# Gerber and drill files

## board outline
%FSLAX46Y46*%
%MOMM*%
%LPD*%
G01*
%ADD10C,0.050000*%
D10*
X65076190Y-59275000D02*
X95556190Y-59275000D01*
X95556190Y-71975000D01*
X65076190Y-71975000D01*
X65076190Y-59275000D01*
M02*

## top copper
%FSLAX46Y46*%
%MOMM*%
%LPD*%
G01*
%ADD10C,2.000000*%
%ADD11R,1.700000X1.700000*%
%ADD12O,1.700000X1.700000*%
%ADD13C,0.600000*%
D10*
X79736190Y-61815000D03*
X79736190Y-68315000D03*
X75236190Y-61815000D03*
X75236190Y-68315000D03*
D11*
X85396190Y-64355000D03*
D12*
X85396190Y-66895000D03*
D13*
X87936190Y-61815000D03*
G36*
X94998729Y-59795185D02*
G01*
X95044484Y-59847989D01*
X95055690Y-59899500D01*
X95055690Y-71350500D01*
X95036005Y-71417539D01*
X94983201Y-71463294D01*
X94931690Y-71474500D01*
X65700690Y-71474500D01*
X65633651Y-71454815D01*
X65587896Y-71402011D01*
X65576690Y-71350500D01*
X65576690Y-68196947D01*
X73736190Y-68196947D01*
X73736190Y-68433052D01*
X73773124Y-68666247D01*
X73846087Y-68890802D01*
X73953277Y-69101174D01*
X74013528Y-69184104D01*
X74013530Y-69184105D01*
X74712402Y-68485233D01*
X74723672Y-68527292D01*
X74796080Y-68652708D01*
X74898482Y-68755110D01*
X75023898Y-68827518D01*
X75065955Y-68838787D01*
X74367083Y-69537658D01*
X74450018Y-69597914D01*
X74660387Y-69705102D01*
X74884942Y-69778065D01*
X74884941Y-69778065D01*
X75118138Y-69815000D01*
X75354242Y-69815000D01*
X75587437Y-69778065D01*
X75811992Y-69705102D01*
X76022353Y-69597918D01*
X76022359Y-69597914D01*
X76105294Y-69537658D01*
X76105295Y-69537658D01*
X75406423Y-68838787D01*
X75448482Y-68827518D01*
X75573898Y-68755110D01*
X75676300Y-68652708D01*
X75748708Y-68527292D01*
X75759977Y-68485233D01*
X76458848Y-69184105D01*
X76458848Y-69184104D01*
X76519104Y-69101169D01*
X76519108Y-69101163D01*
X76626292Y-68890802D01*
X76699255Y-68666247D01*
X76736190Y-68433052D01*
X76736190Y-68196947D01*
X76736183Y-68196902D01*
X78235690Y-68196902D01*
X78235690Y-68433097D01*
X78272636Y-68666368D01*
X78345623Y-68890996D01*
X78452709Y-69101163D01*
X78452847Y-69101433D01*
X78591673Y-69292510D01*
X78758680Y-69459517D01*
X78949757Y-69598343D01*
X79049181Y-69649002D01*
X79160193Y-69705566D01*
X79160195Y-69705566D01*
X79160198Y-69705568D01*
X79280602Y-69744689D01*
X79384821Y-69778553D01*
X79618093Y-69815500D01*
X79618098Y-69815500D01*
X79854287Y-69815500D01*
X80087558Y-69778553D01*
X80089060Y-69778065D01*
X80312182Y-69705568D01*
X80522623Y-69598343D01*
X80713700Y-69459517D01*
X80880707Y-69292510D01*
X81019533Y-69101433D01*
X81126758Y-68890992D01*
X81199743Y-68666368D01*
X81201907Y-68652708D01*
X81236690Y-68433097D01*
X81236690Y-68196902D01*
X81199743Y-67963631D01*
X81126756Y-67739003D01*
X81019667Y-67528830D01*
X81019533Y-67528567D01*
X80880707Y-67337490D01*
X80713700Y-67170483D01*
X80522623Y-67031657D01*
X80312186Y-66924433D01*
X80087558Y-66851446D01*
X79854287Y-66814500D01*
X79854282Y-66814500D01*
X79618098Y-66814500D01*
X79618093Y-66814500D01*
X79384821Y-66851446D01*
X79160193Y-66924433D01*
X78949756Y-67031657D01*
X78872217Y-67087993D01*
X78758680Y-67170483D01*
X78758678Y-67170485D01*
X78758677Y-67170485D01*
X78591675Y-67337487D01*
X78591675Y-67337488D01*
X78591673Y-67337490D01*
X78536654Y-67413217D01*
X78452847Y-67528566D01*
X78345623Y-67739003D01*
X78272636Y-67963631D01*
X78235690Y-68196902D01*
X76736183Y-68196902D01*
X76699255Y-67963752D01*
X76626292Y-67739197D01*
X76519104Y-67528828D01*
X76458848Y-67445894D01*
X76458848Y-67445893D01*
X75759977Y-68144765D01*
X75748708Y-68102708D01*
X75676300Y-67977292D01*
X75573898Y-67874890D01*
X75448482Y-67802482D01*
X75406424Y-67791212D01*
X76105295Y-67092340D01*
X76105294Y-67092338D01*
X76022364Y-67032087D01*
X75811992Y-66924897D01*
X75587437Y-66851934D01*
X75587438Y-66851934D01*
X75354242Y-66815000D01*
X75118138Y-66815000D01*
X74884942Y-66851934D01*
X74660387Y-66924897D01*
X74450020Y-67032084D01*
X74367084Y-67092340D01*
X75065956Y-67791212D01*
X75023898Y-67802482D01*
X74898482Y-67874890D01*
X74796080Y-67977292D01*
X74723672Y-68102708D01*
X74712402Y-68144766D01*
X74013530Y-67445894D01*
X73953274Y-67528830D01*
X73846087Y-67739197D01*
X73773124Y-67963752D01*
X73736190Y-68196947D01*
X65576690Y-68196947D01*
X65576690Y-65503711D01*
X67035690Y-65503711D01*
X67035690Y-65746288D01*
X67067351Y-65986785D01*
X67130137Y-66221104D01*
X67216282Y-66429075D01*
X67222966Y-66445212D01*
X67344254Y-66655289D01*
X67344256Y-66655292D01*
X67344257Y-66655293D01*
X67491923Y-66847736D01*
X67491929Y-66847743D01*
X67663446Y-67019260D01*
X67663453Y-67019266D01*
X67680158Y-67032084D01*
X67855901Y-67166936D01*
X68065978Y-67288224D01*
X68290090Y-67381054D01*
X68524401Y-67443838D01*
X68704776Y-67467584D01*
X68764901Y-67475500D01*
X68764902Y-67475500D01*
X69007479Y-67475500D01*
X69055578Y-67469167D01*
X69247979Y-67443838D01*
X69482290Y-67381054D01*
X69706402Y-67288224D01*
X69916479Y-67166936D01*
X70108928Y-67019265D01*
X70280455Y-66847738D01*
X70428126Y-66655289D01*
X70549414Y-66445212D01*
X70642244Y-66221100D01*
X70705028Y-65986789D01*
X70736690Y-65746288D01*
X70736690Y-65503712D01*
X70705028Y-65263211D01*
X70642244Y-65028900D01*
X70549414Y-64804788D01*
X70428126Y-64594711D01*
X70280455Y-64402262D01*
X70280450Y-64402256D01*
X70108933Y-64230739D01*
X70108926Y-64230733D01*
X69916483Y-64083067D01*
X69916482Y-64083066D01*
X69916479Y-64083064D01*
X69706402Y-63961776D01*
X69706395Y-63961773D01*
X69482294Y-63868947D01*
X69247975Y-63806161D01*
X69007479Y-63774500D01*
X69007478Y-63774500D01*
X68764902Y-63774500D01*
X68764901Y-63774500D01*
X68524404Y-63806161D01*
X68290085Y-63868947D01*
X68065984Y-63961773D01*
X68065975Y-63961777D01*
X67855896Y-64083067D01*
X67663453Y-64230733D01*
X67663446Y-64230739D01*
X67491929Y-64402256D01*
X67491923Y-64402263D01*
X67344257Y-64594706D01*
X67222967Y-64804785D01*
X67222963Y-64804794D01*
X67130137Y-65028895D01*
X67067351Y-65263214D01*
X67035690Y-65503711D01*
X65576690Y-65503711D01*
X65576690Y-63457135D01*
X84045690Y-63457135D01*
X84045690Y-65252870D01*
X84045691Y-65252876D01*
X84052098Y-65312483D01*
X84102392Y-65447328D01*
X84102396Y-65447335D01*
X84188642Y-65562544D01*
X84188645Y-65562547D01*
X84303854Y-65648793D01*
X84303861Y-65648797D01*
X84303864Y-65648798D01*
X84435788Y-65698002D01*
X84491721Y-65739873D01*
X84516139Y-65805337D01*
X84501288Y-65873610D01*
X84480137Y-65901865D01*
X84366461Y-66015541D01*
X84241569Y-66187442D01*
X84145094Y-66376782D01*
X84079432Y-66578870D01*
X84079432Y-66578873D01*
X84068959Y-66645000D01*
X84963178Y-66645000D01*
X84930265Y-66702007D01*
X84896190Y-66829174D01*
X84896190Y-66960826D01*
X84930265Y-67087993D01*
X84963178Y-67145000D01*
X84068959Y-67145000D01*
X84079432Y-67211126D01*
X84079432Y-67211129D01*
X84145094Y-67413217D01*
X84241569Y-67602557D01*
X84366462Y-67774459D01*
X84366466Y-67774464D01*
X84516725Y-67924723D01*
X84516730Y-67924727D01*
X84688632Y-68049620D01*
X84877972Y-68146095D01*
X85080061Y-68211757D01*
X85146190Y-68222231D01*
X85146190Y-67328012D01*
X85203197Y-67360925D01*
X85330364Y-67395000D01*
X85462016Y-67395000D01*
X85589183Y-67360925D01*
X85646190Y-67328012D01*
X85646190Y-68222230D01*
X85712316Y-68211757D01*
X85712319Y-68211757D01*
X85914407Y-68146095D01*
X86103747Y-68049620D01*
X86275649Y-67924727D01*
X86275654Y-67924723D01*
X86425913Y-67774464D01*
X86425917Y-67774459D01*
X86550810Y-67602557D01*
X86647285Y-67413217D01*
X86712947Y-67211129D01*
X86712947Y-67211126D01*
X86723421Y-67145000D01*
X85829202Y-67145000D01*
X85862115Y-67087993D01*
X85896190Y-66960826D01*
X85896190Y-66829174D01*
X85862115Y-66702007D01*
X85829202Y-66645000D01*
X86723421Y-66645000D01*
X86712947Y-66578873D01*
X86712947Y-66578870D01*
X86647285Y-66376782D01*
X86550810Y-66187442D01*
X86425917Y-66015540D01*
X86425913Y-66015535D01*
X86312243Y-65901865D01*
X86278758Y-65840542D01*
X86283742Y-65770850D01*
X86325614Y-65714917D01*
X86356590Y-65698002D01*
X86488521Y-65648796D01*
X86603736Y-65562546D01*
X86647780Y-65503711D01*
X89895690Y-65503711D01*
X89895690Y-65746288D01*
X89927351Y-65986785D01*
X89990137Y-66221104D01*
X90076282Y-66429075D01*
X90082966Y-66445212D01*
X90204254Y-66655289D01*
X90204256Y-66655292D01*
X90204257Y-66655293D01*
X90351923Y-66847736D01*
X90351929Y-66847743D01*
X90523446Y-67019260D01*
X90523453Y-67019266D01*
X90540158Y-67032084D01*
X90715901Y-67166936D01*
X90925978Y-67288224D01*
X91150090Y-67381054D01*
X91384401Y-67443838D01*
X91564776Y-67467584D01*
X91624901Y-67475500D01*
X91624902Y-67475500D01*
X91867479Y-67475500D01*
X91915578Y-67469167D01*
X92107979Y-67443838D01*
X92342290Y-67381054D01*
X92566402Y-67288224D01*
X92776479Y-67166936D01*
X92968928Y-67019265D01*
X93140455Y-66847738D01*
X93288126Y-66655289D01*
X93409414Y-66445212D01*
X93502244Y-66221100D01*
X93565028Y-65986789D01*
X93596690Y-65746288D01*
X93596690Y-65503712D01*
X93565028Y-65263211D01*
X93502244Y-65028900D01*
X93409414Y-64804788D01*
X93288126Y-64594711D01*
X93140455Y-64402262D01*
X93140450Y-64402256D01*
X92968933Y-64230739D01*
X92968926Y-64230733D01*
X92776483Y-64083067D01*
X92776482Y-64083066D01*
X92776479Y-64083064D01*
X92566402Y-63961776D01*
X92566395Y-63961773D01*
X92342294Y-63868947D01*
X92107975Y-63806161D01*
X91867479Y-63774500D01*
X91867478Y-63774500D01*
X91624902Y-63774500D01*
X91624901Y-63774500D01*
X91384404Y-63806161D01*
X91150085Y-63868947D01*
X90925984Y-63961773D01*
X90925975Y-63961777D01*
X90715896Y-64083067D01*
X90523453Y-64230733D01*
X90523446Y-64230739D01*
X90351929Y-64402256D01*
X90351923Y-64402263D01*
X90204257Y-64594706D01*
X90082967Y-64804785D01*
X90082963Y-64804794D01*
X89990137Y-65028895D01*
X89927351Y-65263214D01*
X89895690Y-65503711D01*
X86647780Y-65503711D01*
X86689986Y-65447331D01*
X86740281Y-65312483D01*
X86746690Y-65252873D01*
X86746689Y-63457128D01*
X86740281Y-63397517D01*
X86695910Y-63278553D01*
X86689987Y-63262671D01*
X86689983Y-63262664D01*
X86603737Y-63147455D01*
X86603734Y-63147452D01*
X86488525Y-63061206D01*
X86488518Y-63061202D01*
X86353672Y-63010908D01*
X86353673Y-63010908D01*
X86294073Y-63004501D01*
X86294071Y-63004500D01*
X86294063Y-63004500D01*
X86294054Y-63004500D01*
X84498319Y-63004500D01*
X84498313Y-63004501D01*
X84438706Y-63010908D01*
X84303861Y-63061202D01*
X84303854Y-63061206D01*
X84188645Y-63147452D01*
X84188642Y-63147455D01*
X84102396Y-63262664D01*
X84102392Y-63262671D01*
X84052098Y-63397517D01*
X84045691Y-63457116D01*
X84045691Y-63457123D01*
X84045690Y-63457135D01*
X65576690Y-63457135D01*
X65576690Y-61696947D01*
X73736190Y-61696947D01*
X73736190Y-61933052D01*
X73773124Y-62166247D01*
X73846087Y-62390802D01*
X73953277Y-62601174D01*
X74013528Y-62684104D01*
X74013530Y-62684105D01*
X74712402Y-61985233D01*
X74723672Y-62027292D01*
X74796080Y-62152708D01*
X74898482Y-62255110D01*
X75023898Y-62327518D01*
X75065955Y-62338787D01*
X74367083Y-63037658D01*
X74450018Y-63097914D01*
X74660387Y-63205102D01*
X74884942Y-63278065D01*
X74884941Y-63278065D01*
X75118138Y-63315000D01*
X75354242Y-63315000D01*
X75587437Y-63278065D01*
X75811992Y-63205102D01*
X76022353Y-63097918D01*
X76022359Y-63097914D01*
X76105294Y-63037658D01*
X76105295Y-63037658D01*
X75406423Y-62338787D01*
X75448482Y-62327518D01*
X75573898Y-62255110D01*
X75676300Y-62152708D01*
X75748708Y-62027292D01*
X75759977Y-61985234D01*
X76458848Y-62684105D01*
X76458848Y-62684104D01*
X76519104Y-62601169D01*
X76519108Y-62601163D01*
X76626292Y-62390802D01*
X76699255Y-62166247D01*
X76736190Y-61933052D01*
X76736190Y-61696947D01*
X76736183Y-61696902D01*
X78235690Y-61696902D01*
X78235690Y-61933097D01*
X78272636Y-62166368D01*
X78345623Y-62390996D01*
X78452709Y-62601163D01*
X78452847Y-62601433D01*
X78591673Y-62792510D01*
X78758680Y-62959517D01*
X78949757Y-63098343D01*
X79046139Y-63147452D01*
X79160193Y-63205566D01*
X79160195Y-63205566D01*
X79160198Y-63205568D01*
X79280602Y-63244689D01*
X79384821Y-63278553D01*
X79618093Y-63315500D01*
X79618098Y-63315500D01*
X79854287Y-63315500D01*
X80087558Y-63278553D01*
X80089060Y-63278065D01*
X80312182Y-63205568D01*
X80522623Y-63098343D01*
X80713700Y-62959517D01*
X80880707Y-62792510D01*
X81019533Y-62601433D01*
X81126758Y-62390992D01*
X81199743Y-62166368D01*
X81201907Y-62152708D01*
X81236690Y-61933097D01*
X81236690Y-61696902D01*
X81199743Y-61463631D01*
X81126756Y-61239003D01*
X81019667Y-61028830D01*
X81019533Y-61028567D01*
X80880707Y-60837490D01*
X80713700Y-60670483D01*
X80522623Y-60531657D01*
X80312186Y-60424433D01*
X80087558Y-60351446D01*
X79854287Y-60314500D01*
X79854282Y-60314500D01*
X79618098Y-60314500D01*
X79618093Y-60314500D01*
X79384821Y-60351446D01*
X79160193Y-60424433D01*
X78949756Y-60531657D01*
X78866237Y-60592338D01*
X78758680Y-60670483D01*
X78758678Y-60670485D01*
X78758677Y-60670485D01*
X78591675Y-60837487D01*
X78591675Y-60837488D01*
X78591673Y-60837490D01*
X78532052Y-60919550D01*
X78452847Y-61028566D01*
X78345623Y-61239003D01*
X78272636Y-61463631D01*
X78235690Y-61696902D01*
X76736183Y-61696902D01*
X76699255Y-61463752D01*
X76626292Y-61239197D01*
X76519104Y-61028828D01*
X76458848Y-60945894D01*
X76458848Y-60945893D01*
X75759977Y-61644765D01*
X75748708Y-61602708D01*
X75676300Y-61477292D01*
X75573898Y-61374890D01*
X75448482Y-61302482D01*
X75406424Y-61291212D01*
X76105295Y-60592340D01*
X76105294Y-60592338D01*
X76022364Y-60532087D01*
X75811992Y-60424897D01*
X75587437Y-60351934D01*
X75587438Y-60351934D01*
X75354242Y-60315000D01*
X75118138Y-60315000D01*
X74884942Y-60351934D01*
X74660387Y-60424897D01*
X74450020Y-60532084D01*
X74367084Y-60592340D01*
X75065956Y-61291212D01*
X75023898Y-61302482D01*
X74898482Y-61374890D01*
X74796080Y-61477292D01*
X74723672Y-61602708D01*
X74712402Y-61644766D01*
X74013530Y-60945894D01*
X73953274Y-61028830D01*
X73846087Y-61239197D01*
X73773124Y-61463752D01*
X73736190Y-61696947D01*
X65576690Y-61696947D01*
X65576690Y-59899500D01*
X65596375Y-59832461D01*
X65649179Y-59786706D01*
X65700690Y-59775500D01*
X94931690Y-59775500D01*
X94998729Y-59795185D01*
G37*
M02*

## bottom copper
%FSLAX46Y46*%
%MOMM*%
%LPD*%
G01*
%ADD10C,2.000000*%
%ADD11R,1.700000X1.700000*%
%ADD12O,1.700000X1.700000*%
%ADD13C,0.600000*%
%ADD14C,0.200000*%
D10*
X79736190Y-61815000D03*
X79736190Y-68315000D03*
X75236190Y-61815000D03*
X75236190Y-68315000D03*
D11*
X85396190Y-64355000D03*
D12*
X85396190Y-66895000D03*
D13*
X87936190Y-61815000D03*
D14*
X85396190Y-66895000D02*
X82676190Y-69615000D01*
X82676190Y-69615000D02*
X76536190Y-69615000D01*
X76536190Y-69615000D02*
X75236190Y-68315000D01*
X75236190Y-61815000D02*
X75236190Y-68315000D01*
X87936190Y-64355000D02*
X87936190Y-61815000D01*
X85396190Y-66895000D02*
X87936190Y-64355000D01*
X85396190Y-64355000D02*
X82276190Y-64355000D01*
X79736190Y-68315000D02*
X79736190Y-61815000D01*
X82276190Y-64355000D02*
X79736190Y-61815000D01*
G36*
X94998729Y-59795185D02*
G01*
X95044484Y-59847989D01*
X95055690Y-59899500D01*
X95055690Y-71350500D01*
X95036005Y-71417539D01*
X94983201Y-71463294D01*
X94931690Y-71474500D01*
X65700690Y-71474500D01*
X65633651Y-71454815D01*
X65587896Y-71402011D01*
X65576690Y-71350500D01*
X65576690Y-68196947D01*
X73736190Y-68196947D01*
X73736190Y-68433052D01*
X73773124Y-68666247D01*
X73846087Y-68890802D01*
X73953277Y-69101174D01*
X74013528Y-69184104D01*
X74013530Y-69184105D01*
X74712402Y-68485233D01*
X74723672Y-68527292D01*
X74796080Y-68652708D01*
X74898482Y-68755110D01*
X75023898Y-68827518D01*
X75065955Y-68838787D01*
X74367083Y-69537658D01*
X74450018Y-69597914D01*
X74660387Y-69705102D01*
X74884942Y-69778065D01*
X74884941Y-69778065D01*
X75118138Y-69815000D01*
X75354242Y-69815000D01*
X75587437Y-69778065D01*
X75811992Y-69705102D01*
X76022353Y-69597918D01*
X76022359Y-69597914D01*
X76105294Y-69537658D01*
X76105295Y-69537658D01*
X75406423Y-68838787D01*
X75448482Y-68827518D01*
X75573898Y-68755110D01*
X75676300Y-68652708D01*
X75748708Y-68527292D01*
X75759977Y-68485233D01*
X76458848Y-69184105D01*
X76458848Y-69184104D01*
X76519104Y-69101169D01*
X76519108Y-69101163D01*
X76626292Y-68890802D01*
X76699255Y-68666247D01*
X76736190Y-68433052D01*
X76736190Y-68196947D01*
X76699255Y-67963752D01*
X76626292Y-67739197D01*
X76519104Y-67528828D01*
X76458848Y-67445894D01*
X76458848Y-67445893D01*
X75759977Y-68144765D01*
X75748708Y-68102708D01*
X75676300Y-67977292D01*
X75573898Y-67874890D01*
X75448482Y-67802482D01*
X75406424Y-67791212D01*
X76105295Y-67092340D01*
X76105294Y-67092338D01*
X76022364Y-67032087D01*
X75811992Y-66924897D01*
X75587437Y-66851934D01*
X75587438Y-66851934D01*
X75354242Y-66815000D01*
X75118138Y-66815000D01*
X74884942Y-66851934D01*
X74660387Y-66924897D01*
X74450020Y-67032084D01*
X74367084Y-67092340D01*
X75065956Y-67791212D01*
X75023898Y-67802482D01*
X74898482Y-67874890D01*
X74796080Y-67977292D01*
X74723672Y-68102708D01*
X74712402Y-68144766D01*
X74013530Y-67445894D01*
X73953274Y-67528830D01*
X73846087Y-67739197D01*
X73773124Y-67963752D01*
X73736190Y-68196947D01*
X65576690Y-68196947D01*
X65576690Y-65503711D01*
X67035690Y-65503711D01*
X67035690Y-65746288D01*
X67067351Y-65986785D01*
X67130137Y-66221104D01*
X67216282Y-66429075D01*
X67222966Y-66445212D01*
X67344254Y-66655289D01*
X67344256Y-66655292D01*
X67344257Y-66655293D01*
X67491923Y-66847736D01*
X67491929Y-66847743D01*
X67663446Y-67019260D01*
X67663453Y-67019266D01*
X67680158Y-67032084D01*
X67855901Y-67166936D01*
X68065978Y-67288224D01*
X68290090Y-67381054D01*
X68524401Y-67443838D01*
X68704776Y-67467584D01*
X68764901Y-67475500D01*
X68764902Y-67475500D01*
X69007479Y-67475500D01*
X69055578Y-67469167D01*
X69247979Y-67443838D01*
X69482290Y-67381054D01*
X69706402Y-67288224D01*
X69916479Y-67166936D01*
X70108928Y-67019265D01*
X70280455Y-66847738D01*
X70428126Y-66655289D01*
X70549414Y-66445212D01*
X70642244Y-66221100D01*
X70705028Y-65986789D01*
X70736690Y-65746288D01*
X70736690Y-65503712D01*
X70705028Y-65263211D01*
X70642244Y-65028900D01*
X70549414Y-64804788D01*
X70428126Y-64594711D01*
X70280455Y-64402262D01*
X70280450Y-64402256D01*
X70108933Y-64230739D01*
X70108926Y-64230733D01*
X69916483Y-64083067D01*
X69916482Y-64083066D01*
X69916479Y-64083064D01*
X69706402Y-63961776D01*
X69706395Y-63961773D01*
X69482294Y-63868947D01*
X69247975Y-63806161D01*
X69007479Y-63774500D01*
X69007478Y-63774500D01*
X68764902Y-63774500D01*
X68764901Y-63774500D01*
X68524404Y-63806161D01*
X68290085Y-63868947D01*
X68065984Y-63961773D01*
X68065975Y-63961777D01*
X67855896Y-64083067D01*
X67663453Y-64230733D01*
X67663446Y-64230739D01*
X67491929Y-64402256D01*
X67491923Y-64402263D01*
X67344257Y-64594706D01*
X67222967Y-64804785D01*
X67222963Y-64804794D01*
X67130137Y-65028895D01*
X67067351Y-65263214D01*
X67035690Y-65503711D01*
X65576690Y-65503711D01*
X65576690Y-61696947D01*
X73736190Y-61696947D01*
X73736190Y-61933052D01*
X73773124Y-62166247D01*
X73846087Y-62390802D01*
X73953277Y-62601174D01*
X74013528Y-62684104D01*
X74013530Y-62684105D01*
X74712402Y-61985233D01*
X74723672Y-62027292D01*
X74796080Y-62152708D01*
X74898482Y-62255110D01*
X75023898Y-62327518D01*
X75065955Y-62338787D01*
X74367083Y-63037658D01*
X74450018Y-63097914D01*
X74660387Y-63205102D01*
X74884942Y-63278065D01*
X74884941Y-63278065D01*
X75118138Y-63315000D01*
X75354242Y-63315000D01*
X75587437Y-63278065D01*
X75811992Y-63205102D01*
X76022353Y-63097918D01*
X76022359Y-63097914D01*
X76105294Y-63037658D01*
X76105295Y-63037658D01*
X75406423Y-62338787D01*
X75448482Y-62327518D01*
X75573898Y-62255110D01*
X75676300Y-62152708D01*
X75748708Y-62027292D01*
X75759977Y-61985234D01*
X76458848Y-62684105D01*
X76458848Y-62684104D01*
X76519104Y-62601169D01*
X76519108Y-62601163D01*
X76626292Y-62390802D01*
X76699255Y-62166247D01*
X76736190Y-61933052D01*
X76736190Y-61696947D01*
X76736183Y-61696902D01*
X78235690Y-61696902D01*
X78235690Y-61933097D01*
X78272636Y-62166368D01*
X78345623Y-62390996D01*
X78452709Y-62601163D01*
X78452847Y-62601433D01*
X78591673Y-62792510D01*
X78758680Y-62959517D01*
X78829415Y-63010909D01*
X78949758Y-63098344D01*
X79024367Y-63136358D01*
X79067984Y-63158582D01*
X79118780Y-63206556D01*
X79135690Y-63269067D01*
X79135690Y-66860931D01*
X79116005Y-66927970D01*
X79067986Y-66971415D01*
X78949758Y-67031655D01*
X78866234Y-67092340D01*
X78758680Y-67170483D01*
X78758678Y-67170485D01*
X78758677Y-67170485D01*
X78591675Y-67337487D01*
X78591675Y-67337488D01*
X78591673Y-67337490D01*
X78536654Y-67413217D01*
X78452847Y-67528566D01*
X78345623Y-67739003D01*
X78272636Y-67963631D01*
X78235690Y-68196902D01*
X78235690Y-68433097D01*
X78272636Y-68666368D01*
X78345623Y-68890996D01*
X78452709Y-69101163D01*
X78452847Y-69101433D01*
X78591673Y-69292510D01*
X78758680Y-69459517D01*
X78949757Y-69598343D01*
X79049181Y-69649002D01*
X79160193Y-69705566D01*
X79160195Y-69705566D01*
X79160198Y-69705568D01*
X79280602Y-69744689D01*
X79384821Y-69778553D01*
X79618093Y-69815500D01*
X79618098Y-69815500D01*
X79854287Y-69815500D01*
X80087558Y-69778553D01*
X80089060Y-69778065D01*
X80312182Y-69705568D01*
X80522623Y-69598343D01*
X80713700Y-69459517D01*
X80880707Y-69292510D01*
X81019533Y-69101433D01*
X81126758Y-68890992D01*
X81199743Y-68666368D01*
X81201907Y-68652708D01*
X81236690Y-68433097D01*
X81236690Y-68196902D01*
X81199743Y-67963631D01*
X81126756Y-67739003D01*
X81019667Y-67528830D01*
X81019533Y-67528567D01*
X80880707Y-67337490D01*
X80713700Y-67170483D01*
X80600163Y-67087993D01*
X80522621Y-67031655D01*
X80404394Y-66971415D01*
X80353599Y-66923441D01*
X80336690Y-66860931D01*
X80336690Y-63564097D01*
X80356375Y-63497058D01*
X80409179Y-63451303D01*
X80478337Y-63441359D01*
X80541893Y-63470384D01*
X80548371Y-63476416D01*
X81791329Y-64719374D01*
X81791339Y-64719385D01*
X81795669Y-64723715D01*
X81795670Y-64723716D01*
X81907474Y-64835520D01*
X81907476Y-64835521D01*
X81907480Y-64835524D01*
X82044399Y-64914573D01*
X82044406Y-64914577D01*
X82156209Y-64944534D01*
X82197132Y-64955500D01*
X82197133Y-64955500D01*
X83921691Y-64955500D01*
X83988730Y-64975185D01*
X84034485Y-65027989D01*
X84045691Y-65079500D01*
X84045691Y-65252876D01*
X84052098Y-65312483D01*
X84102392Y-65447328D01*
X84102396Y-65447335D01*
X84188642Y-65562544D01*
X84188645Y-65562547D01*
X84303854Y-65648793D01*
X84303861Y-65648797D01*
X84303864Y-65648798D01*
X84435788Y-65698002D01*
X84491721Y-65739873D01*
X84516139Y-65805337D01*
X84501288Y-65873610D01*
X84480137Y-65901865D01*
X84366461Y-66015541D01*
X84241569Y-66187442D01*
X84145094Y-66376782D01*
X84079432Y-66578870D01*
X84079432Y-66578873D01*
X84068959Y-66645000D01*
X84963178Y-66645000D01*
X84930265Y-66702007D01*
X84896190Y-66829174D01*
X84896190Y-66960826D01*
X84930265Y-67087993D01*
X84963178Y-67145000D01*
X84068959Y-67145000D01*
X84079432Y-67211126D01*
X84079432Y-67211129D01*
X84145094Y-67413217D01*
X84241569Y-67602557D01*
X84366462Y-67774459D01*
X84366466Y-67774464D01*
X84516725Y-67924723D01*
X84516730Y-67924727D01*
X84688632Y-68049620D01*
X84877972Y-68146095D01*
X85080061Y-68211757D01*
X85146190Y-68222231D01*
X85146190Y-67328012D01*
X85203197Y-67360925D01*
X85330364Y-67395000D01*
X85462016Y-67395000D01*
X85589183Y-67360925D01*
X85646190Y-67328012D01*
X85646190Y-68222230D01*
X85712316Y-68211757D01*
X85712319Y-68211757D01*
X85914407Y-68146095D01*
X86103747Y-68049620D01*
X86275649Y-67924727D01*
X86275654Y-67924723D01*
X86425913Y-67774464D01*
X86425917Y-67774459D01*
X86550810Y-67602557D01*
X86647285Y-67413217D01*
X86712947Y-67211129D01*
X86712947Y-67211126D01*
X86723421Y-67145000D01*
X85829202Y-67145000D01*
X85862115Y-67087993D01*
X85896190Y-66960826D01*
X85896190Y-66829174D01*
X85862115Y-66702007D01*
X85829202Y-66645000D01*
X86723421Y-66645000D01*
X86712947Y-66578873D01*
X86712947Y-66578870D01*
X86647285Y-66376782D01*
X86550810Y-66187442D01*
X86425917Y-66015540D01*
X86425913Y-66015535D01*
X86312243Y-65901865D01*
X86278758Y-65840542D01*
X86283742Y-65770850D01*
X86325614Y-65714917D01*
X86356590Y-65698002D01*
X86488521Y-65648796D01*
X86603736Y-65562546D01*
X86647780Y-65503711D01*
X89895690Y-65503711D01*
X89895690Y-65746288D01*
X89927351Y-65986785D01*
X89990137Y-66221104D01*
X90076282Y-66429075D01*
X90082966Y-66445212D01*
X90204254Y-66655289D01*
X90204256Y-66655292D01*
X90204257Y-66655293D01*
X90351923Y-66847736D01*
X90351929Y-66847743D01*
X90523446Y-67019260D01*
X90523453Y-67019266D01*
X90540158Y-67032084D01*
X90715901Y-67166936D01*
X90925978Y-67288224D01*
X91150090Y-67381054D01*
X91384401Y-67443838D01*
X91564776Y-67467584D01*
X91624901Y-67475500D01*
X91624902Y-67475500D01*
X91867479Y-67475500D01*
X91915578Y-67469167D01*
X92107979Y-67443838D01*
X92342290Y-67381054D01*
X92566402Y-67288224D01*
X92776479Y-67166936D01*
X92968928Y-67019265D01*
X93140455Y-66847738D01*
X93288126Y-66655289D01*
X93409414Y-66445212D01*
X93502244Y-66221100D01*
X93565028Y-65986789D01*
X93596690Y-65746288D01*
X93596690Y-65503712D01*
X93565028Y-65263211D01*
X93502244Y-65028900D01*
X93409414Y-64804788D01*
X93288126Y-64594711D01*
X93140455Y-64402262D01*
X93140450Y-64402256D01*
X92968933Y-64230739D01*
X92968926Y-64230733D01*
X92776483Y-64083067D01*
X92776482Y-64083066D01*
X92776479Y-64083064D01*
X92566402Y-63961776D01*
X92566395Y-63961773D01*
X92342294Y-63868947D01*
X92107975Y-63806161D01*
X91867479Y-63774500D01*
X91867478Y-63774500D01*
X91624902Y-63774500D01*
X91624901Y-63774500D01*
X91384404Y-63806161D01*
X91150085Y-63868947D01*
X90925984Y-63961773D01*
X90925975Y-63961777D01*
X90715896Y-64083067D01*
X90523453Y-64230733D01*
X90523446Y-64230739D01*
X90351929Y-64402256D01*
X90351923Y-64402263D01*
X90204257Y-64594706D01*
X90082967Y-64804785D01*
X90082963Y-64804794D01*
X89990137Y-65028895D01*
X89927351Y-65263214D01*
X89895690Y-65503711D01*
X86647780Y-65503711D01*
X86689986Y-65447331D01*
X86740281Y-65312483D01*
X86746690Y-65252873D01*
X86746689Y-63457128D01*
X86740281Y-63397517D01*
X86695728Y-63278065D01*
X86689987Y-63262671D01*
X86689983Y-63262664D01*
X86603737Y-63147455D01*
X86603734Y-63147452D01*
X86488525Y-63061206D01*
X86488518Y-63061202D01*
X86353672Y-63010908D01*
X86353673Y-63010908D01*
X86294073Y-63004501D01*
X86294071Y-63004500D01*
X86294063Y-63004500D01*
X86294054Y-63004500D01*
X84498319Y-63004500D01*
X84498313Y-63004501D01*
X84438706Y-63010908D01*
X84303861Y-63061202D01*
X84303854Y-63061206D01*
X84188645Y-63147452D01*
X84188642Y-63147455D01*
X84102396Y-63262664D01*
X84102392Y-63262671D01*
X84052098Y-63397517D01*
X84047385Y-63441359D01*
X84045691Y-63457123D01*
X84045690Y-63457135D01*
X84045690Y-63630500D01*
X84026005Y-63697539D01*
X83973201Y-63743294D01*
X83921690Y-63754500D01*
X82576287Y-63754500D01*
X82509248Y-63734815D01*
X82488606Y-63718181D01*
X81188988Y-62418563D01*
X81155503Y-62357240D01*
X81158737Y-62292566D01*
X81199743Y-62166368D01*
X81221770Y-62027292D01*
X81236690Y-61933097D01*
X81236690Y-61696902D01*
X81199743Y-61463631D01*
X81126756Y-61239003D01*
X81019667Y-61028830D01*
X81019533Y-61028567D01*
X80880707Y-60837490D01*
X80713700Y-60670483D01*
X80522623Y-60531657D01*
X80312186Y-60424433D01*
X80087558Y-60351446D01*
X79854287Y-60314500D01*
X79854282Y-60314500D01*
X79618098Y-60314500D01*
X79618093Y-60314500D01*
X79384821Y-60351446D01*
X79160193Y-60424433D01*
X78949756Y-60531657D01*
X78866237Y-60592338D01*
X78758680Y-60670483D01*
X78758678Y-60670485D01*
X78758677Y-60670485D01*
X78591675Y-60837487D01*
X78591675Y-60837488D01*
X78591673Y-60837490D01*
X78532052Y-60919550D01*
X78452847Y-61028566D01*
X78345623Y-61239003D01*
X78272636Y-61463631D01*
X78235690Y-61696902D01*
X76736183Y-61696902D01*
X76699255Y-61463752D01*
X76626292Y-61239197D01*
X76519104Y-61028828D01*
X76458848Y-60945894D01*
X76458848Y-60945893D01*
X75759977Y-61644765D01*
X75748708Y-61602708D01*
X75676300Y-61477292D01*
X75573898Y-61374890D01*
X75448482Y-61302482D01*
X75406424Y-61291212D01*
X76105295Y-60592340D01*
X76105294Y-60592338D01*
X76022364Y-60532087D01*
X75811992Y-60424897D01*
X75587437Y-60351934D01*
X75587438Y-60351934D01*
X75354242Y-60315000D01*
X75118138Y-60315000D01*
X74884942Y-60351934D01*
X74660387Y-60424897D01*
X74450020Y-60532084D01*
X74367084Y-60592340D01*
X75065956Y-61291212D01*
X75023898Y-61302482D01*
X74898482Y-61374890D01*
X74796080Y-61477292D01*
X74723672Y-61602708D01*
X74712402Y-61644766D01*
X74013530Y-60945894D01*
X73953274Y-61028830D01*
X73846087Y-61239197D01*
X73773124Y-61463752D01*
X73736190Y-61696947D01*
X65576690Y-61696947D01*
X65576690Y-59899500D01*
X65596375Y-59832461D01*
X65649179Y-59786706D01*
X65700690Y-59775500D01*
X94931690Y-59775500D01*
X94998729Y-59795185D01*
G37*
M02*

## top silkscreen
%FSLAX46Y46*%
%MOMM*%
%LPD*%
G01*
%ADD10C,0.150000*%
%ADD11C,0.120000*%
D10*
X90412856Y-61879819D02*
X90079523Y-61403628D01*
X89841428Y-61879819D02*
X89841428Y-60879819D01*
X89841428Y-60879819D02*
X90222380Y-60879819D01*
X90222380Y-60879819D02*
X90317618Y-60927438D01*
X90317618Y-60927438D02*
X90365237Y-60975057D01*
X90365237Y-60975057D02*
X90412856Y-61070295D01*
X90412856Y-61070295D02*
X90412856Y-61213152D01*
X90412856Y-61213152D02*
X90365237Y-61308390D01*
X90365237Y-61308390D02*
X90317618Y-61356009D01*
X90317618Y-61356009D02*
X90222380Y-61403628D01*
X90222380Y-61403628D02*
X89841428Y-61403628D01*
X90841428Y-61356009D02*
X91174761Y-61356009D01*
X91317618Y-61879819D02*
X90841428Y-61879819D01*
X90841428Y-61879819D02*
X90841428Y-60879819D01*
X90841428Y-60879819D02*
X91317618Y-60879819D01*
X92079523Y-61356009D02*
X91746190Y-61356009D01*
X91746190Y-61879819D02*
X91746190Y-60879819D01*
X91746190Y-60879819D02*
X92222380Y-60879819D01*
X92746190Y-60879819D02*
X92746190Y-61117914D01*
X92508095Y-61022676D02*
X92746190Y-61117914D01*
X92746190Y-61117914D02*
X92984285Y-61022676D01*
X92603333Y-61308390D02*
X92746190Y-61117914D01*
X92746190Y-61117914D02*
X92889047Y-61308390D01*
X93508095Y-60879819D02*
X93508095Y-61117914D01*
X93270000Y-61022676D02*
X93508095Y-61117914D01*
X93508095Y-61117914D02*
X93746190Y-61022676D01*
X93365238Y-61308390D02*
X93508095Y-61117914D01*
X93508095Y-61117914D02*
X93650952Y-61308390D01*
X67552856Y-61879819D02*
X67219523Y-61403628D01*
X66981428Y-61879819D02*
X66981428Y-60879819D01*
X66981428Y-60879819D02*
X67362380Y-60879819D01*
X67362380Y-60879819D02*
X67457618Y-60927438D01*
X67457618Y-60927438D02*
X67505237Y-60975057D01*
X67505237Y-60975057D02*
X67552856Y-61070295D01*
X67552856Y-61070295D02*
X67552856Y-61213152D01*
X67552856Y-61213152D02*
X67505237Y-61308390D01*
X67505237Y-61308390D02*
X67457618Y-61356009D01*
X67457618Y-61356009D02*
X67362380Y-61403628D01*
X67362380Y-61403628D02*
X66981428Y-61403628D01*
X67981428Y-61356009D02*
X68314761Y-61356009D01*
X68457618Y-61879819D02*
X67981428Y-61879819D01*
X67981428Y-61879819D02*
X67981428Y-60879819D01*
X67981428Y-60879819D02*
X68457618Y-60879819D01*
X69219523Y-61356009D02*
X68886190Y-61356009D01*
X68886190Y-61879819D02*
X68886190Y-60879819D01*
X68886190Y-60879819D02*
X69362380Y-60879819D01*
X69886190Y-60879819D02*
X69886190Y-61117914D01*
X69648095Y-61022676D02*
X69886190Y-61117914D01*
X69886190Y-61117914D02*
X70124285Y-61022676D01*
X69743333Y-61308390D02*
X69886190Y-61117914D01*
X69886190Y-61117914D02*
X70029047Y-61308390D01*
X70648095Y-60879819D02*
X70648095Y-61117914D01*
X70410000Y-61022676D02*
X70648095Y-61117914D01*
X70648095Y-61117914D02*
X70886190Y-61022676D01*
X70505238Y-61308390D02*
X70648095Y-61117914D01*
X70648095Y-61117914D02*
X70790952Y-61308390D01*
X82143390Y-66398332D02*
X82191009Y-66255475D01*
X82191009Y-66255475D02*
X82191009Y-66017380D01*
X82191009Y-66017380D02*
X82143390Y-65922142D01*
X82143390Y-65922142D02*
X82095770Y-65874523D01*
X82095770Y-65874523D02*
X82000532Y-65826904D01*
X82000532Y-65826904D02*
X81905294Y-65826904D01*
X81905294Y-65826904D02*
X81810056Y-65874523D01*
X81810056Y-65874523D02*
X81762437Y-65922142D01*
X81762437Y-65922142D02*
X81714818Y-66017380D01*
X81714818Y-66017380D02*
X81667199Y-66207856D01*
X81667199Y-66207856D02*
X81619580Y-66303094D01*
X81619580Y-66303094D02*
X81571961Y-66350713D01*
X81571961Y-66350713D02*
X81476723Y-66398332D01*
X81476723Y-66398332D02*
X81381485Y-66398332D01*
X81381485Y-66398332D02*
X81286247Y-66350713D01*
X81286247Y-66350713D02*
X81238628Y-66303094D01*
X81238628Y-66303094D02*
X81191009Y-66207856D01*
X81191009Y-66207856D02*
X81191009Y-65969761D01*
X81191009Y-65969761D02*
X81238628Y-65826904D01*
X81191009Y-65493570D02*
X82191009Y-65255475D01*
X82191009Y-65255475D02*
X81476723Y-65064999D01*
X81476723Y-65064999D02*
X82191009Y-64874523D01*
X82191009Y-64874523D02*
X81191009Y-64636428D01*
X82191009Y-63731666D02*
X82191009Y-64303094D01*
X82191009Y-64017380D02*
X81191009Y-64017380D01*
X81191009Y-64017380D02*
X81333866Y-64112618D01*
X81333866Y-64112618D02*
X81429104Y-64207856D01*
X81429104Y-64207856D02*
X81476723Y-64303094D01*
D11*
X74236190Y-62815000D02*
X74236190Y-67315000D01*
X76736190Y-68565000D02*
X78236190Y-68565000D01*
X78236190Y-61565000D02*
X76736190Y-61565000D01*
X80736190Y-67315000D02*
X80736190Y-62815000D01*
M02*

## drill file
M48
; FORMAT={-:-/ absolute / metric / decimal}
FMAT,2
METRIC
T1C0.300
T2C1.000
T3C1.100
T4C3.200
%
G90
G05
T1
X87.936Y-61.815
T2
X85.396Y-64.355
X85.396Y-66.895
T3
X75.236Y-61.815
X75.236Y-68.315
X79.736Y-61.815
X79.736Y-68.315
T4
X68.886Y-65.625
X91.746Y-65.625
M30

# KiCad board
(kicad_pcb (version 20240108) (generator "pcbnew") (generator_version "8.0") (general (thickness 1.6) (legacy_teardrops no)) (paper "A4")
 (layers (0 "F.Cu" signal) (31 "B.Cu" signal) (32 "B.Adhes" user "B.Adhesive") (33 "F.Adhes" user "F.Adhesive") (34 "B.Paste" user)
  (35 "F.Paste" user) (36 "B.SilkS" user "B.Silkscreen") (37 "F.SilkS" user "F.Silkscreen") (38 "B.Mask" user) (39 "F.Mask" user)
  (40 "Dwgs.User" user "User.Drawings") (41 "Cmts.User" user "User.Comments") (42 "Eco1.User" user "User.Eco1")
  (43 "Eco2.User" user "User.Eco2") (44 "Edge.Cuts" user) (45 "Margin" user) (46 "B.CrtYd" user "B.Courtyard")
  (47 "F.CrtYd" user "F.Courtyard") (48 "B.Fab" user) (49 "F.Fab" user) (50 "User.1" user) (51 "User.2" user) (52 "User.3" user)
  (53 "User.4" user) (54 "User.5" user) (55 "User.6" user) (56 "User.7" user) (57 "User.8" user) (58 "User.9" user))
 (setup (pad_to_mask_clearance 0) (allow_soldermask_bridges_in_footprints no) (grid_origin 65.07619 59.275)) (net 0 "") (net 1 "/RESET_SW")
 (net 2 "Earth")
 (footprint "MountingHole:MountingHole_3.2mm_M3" (layer "F.Cu") (at 91.74619 65.625)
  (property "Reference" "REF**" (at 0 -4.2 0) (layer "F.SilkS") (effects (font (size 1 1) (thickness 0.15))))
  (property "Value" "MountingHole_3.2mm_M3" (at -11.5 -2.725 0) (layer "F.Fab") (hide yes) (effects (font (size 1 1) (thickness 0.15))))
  (pad "" np_thru_hole circle (at 0 0) (size 3.2 3.2) (drill 3.2) (layers "*.Cu" "*.Mask")))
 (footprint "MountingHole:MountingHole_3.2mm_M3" (layer "F.Cu") (at 68.88619 65.625)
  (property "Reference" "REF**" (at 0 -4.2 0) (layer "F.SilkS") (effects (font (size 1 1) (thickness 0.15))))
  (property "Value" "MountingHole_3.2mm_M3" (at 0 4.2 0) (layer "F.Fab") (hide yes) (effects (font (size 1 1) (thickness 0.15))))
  (pad "" np_thru_hole circle (at 0 0) (size 3.2 3.2) (drill 3.2) (layers "*.Cu" "*.Mask")))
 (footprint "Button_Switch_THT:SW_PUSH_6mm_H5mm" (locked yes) (layer "F.Cu") (at 79.73619 61.815 -90)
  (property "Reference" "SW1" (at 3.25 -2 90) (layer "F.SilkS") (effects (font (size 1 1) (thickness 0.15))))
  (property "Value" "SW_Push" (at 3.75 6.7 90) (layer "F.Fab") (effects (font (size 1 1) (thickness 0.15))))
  (fp_line (start 1 5.5) (end 5.5 5.5) (stroke (width 0.12) (type solid)) (layer "F.SilkS"))
  (fp_line (start 6.75 3) (end 6.75 1.5) (stroke (width 0.12) (type solid)) (layer "F.SilkS"))
  (fp_line (start -0.25 1.5) (end -0.25 3) (stroke (width 0.12) (type solid)) (layer "F.SilkS"))
  (fp_line (start 5.5 -1) (end 1 -1) (stroke (width 0.12) (type solid)) (layer "F.SilkS"))
  (pad "1" thru_hole circle (at 0 0) (size 2 2) (drill 1.1) (layers "*.Cu" "*.Mask") (remove_unused_layers no) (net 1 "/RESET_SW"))
  (pad "1" thru_hole circle (at 6.5 0) (size 2 2) (drill 1.1) (layers "*.Cu" "*.Mask") (remove_unused_layers no) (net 1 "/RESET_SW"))
  (pad "2" thru_hole circle (at 0 4.5) (size 2 2) (drill 1.1) (layers "*.Cu" "*.Mask") (remove_unused_layers no) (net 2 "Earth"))
  (pad "2" thru_hole circle (at 6.5 4.5) (size 2 2) (drill 1.1) (layers "*.Cu" "*.Mask") (remove_unused_layers no) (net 2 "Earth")))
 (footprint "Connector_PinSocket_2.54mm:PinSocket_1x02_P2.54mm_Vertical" (layer "B.Cu") (at 85.39619 64.355 180)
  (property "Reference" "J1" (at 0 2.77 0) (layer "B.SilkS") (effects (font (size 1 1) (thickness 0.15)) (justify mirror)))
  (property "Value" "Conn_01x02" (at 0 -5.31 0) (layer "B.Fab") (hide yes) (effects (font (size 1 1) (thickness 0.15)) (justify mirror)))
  (pad "1" thru_hole rect (at 0 0 180) (size 1.7 1.7) (drill 1) (layers "*.Cu" "*.Mask") (remove_unused_layers no) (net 1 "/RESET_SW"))
  (pad "2" thru_hole oval (at 0 -2.54 180) (size 1.7 1.7) (drill 1) (layers "*.Cu" "*.Mask") (remove_unused_layers no) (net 2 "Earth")))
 (gr_rect (start 65.07619 59.275) (end 95.55619 71.975) (stroke (width 0.05) (type default)) (fill none) (layer "Edge.Cuts"))
 (via (at 87.93619 61.815) (size 0.6) (drill 0.3) (layers "F.Cu" "B.Cu") (free yes) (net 2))
 (segment (start 85.39619 66.895) (end 82.67619 69.615) (width 0.2) (layer "B.Cu") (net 2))
 (segment (start 82.67619 69.615) (end 76.53619 69.615) (width 0.2) (layer "B.Cu") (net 2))
 (segment (start 76.53619 69.615) (end 75.23619 68.315) (width 0.2) (layer "B.Cu") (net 2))
 (segment (start 75.23619 61.815) (end 75.23619 68.315) (width 0.2) (layer "B.Cu") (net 2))
 (segment (start 87.93619 64.355) (end 87.93619 61.815) (width 0.2) (layer "B.Cu") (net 2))
 (segment (start 85.39619 66.895) (end 87.93619 64.355) (width 0.2) (layer "B.Cu") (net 2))
 (segment (start 85.39619 64.355) (end 82.27619 64.355) (width 0.2) (layer "B.Cu") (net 1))
 (segment (start 79.73619 68.315) (end 79.73619 61.815) (width 0.2) (layer "B.Cu") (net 1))
 (segment (start 82.27619 64.355) (end 79.73619 61.815) (width 0.2) (layer "B.Cu") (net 1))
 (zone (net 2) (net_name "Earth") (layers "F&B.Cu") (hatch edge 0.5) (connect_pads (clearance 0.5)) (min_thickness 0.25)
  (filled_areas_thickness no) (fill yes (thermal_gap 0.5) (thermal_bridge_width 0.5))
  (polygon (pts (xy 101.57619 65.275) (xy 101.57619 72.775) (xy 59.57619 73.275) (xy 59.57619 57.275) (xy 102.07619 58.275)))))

